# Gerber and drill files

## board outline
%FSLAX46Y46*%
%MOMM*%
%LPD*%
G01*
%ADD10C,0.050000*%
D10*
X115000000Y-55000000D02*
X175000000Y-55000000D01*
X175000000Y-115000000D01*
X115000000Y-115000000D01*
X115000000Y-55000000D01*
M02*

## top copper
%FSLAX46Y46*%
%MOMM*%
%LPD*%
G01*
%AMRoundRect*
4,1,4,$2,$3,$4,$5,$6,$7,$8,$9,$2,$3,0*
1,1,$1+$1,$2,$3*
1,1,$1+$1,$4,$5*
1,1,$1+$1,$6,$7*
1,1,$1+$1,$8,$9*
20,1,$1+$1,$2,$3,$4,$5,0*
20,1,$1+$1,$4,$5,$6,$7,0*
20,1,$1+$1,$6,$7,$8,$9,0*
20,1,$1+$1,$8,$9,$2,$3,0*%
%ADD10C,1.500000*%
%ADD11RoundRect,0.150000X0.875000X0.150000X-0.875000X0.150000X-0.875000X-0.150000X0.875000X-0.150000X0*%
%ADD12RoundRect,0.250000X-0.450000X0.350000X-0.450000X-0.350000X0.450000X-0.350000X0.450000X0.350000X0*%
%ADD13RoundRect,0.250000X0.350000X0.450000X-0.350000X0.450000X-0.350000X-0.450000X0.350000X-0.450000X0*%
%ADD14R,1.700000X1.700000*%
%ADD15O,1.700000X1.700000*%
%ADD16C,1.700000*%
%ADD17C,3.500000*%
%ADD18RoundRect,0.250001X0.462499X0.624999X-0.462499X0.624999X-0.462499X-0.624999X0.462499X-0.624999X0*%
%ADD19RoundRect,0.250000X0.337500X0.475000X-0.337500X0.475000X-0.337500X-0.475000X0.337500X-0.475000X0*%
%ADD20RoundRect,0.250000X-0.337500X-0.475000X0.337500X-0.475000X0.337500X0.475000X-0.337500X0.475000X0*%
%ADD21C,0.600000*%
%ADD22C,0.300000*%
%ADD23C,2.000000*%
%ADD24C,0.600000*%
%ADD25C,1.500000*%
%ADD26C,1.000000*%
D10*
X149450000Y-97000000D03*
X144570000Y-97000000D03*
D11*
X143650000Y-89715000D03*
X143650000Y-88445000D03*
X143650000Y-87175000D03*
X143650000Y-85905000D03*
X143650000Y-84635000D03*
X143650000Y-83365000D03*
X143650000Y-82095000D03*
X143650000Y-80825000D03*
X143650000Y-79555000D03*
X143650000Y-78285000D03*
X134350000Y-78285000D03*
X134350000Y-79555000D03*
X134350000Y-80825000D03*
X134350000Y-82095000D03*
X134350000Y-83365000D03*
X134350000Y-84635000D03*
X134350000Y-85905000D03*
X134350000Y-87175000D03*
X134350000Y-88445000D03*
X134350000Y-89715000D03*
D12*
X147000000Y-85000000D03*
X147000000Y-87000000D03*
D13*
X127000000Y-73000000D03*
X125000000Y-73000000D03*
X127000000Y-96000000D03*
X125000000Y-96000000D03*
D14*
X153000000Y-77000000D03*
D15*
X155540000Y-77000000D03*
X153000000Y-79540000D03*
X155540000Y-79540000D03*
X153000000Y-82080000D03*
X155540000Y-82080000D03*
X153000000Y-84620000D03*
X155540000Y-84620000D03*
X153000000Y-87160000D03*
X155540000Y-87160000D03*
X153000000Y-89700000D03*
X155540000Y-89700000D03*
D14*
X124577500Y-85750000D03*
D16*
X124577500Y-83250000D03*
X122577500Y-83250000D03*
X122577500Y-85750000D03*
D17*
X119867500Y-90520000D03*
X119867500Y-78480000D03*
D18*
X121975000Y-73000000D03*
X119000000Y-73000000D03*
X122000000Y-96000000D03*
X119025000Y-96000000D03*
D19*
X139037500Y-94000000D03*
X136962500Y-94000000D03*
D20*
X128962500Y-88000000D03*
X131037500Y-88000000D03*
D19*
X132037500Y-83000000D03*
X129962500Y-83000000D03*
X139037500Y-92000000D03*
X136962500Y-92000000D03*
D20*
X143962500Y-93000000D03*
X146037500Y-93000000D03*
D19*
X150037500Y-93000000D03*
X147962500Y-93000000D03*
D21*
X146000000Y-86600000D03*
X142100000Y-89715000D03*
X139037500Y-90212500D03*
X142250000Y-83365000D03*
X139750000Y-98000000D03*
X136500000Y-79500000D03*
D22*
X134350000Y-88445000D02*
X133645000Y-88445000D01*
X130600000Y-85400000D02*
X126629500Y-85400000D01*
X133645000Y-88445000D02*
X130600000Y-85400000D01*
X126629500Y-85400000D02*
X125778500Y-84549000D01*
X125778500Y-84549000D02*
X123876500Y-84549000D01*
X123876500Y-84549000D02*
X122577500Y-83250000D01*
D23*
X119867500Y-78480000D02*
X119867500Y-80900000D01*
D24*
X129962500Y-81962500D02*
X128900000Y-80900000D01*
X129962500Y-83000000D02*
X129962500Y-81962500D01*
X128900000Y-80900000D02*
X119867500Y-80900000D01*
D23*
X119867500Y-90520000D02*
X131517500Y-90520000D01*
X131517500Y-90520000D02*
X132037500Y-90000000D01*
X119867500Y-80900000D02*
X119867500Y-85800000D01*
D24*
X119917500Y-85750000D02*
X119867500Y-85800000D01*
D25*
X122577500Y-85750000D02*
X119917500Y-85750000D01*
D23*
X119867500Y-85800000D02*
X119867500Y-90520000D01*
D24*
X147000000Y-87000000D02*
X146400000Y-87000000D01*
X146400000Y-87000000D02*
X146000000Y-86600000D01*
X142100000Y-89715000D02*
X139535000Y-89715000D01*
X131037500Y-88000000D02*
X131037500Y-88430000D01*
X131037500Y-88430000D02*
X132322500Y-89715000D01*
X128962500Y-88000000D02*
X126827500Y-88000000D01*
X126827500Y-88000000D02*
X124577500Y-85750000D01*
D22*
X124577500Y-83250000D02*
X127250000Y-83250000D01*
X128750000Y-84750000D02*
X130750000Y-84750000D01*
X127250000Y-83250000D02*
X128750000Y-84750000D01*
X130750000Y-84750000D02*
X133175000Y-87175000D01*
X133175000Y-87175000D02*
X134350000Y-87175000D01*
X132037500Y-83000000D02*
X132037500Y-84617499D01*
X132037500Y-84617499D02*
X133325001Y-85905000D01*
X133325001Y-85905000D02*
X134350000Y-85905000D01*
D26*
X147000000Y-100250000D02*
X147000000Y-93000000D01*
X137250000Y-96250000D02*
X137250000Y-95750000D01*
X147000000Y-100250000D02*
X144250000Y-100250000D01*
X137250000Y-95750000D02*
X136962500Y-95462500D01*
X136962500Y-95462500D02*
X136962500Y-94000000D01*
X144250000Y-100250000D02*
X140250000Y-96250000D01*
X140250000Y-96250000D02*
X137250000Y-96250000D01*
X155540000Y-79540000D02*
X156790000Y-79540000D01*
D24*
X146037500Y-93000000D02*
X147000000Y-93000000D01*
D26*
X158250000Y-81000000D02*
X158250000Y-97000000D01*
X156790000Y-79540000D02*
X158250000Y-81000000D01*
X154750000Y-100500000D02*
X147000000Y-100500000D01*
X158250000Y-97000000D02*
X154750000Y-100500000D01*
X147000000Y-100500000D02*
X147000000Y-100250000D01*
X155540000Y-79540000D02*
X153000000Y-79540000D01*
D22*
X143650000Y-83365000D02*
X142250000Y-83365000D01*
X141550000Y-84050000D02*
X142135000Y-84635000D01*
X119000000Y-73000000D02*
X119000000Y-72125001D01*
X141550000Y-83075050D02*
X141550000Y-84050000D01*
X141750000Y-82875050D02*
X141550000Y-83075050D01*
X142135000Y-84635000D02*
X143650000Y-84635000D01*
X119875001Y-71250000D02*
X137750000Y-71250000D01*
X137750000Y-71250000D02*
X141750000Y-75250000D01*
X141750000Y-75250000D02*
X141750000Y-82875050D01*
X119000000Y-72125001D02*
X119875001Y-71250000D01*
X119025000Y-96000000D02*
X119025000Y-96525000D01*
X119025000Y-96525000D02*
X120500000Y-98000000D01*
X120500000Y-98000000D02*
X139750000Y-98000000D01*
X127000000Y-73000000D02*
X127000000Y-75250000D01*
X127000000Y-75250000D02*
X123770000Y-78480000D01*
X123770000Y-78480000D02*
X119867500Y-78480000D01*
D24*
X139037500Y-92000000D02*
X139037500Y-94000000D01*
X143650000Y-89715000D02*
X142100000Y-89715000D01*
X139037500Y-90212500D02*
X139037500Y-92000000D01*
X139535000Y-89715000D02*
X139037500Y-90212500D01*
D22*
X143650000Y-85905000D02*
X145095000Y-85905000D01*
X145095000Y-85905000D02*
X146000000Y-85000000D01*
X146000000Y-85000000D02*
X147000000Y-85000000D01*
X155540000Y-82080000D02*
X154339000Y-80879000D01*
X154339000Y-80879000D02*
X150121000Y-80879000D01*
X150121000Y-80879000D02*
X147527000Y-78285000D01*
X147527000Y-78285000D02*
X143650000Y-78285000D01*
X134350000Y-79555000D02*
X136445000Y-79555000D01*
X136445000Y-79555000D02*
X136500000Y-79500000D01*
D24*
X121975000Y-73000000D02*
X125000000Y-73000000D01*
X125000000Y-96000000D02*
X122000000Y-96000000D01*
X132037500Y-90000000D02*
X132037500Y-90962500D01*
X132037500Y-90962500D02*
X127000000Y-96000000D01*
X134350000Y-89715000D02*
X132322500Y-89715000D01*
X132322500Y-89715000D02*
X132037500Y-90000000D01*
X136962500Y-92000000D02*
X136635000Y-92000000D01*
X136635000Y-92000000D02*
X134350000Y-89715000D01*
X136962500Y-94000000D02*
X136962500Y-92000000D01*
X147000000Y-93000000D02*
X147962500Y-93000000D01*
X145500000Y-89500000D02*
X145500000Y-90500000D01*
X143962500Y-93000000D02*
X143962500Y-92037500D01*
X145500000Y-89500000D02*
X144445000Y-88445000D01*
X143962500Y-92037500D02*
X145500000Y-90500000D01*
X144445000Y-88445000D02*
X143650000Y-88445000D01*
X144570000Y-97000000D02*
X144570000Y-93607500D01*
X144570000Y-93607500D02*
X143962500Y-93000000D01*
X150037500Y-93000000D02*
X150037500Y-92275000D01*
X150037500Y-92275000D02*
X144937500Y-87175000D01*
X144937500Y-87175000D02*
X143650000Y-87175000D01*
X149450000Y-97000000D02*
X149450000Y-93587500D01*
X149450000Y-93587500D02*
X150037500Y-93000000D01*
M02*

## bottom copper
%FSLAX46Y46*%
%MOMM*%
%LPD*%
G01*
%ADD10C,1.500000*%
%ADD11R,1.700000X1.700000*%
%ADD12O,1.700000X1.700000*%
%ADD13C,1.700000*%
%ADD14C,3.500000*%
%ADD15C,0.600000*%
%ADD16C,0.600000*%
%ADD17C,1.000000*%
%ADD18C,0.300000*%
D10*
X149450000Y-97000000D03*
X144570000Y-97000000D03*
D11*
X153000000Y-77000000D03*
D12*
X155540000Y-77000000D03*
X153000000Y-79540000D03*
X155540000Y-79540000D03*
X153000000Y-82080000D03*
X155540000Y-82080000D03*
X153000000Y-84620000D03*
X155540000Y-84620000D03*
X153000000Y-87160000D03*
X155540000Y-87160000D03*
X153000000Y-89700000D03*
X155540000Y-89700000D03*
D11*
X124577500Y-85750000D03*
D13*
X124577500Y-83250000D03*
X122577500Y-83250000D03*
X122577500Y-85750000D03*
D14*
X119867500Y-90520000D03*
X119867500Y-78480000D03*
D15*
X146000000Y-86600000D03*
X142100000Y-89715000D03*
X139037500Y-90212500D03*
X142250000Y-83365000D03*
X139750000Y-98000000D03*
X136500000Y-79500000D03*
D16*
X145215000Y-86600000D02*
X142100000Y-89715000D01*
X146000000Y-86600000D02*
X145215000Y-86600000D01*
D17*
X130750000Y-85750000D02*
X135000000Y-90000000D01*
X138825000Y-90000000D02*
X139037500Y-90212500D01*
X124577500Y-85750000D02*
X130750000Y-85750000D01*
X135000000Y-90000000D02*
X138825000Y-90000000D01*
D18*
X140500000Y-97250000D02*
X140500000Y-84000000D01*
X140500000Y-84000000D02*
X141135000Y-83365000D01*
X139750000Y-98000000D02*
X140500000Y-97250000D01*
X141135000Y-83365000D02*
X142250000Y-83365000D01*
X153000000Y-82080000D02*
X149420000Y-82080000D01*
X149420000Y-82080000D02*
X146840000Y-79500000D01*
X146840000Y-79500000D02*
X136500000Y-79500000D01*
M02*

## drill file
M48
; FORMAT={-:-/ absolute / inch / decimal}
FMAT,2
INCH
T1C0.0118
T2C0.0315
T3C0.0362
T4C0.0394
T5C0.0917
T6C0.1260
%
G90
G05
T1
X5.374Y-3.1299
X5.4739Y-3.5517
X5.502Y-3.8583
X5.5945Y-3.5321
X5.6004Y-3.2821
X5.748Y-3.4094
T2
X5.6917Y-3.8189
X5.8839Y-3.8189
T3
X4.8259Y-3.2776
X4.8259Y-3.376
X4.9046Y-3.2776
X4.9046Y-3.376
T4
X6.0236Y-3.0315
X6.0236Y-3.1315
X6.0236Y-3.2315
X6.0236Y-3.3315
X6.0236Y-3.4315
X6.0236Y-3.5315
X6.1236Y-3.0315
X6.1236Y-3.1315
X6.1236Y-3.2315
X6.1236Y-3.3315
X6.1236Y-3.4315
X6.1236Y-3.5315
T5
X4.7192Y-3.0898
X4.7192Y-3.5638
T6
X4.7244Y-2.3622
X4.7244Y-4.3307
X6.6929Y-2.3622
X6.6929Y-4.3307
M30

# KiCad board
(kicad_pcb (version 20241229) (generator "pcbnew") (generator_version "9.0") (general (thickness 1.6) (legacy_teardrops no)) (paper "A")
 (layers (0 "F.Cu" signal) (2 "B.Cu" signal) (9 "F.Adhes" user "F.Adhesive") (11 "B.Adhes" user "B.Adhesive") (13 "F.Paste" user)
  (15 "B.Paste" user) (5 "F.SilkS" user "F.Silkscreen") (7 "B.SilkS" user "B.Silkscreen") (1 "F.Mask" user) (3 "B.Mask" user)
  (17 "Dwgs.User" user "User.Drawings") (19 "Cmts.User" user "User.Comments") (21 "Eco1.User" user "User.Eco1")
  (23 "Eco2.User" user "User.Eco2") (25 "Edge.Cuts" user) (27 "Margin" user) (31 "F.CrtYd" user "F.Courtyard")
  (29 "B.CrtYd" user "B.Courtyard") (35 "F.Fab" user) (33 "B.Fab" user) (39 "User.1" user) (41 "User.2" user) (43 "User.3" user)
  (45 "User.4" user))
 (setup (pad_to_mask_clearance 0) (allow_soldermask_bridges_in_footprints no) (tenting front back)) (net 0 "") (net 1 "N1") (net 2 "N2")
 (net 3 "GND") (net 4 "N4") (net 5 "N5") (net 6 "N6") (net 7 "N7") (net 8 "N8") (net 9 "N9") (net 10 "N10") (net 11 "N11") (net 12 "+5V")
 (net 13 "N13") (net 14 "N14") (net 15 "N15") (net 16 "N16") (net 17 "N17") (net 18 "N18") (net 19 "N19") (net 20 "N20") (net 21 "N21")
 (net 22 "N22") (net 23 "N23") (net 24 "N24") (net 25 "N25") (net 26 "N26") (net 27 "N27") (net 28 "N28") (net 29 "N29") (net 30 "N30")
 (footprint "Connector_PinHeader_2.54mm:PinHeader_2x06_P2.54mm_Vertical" (layer "F.Cu") (at 153 77)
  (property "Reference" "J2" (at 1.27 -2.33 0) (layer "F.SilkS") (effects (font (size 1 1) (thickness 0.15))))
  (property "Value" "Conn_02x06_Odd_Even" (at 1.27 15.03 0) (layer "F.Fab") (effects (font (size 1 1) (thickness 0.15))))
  (pad "1" thru_hole rect (at 0 0) (size 1.7 1.7) (drill 1) (layers "*.Cu" "*.Mask") (remove_unused_layers no) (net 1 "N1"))
  (pad "2" thru_hole oval (at 2.54 0) (size 1.7 1.7) (drill 1) (layers "*.Cu" "*.Mask") (remove_unused_layers no) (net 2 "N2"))
  (pad "3" thru_hole oval (at 0 2.54) (size 1.7 1.7) (drill 1) (layers "*.Cu" "*.Mask") (remove_unused_layers no) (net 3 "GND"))
  (pad "4" thru_hole oval (at 2.54 2.54) (size 1.7 1.7) (drill 1) (layers "*.Cu" "*.Mask") (remove_unused_layers no) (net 3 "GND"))
  (pad "5" thru_hole oval (at 0 5.08) (size 1.7 1.7) (drill 1) (layers "*.Cu" "*.Mask") (remove_unused_layers no) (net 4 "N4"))
  (pad "6" thru_hole oval (at 2.54 5.08) (size 1.7 1.7) (drill 1) (layers "*.Cu" "*.Mask") (remove_unused_layers no) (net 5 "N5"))
  (pad "7" thru_hole oval (at 0 7.62) (size 1.7 1.7) (drill 1) (layers "*.Cu" "*.Mask") (remove_unused_layers no) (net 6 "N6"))
  (pad "8" thru_hole oval (at 2.54 7.62) (size 1.7 1.7) (drill 1) (layers "*.Cu" "*.Mask") (remove_unused_layers no) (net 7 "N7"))
  (pad "9" thru_hole oval (at 0 10.16) (size 1.7 1.7) (drill 1) (layers "*.Cu" "*.Mask") (remove_unused_layers no) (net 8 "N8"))
  (pad "10" thru_hole oval (at 2.54 10.16) (size 1.7 1.7) (drill 1) (layers "*.Cu" "*.Mask") (remove_unused_layers no) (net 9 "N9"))
  (pad "11" thru_hole oval (at 0 12.7) (size 1.7 1.7) (drill 1) (layers "*.Cu" "*.Mask") (remove_unused_layers no) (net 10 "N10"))
  (pad "12" thru_hole oval (at 2.54 12.7) (size 1.7 1.7) (drill 1) (layers "*.Cu" "*.Mask") (remove_unused_layers no) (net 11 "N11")))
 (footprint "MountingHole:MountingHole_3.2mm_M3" (layer "F.Cu") (at 120 110)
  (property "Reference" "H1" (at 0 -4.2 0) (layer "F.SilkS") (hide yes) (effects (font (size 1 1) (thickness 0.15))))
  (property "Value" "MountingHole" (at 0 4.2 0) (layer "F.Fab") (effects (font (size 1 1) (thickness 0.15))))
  (pad "" np_thru_hole circle (at 0 0) (size 3.2 3.2) (drill 3.2) (layers "*.Cu" "*.Mask")))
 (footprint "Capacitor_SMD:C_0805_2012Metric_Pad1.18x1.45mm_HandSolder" (layer "F.Cu") (at 130 88)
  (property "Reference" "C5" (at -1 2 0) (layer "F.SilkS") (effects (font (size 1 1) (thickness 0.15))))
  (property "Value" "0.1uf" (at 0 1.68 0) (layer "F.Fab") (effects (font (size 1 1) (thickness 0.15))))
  (pad "1" smd roundrect (at -1.0375 0) (size 1.175 1.45) (layers "F.Cu" "F.Mask" "F.Paste") (roundrect_rratio 0.212766) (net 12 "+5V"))
  (pad "2" smd roundrect (at 1.0375 0) (size 1.175 1.45) (layers "F.Cu" "F.Mask" "F.Paste") (roundrect_rratio 0.212766) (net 3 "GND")))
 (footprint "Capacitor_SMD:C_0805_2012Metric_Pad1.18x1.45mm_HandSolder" (layer "F.Cu") (at 138 94 180)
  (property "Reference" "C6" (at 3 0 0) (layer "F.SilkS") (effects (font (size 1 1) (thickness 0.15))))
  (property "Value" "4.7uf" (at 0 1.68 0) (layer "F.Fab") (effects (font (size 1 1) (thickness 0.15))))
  (pad "1" smd roundrect (at -1.0375 0 180) (size 1.175 1.45) (layers "F.Cu" "F.Mask" "F.Paste") (roundrect_rratio 0.212766) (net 12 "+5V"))
  (pad "2" smd roundrect (at 1.0375 0 180) (size 1.175 1.45) (layers "F.Cu" "F.Mask" "F.Paste") (roundrect_rratio 0.212766) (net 3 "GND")))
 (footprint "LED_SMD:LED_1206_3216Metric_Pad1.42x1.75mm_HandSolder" (layer "F.Cu") (at 120.5125 96 180)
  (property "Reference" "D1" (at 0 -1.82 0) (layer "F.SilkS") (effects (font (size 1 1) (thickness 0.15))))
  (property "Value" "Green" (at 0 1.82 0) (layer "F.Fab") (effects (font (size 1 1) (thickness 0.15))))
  (pad "1" smd roundrect (at -1.4875 0 180) (size 1.425 1.75) (layers "F.Cu" "F.Mask" "F.Paste") (roundrect_rratio 0.175439) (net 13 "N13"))
  (pad "2" smd roundrect (at 1.4875 0 180) (size 1.425 1.75) (layers "F.Cu" "F.Mask" "F.Paste") (roundrect_rratio 0.175439) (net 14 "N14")))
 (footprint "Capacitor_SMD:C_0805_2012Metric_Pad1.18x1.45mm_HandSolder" (layer "F.Cu") (at 138 92 180)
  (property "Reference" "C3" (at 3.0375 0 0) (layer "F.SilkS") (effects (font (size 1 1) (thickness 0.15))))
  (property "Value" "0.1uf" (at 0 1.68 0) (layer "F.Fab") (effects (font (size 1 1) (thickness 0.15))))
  (pad "1" smd roundrect (at -1.0375 0 180) (size 1.175 1.45) (layers "F.Cu" "F.Mask" "F.Paste") (roundrect_rratio 0.212766) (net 12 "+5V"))
  (pad "2" smd roundrect (at 1.0375 0 180) (size 1.175 1.45) (layers "F.Cu" "F.Mask" "F.Paste") (roundrect_rratio 0.212766) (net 3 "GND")))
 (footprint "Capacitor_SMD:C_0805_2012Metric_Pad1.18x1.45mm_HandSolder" (layer "F.Cu") (at 131 83 180)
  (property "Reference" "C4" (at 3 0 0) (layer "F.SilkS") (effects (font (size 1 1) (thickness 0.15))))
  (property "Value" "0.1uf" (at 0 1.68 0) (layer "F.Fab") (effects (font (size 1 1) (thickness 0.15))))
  (pad "1" smd roundrect (at -1.0375 0 180) (size 1.175 1.45) (layers "F.Cu" "F.Mask" "F.Paste") (roundrect_rratio 0.212766) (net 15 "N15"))
  (pad "2" smd roundrect (at 1.0375 0 180) (size 1.175 1.45) (layers "F.Cu" "F.Mask" "F.Paste") (roundrect_rratio 0.212766) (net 3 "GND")))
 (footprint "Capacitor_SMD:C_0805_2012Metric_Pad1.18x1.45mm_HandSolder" (layer "F.Cu") (at 145 93)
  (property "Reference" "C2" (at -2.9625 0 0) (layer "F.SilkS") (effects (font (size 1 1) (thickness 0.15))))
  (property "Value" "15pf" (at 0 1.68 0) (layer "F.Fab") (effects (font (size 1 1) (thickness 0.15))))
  (pad "1" smd roundrect (at -1.0375 0) (size 1.175 1.45) (layers "F.Cu" "F.Mask" "F.Paste") (roundrect_rratio 0.212766) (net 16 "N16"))
  (pad "2" smd roundrect (at 1.0375 0) (size 1.175 1.45) (layers "F.Cu" "F.Mask" "F.Paste") (roundrect_rratio 0.212766) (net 3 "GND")))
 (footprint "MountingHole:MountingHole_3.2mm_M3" (layer "F.Cu") (at 170 110)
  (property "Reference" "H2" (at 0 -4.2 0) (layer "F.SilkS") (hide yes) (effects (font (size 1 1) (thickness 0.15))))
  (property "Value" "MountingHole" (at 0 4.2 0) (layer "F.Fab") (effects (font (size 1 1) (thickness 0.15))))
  (pad "" np_thru_hole circle (at 0 0) (size 3.2 3.2) (drill 3.2) (layers "*.Cu" "*.Mask")))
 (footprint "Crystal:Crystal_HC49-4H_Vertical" (layer "F.Cu") (at 149.45 97 180)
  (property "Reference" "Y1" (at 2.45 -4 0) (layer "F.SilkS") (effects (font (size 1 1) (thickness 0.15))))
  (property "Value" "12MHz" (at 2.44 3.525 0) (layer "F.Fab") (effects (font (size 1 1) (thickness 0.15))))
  (pad "1" thru_hole circle (at 0 0 180) (size 1.5 1.5) (drill 0.8) (layers "*.Cu" "*.Mask") (remove_unused_layers no) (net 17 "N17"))
  (pad "2" thru_hole circle (at 4.88 0 180) (size 1.5 1.5) (drill 0.8) (layers "*.Cu" "*.Mask") (remove_unused_layers no) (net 16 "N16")))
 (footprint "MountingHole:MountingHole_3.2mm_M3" (layer "F.Cu") (at 170 60)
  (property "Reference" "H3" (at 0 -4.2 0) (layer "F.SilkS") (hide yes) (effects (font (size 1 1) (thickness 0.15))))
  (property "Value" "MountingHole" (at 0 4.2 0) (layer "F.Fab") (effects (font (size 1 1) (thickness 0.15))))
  (pad "" np_thru_hole circle (at 0 0) (size 3.2 3.2) (drill 3.2) (layers "*.Cu" "*.Mask")))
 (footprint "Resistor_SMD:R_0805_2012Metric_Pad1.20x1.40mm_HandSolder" (layer "F.Cu") (at 126 73 180)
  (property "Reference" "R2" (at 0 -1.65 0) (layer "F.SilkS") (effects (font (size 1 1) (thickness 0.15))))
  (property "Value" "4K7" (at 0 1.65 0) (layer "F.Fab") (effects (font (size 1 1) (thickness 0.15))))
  (pad "1" smd roundrect (at -1 0 180) (size 1.2 1.4) (layers "F.Cu" "F.Mask" "F.Paste") (roundrect_rratio 0.208333) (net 3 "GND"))
  (pad "2" smd roundrect (at 1 0 180) (size 1.2 1.4) (layers "F.Cu" "F.Mask" "F.Paste") (roundrect_rratio 0.208333) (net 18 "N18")))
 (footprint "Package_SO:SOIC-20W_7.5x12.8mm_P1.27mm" (layer "F.Cu") (at 139 84 180)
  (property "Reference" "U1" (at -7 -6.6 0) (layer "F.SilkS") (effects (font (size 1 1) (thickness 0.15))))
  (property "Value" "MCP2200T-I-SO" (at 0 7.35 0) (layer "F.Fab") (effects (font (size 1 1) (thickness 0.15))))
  (pad "1" smd roundrect (at -4.65 -5.715 180) (size 2.05 0.6) (layers "F.Cu" "F.Mask" "F.Paste") (roundrect_rratio 0.25) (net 12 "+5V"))
  (pad "2" smd roundrect (at -4.65 -4.445 180) (size 2.05 0.6) (layers "F.Cu" "F.Mask" "F.Paste") (roundrect_rratio 0.25) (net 16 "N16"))
  (pad "3" smd roundrect (at -4.65 -3.175 180) (size 2.05 0.6) (layers "F.Cu" "F.Mask" "F.Paste") (roundrect_rratio 0.25) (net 17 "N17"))
  (pad "4" smd roundrect (at -4.65 -1.905 180) (size 2.05 0.6) (layers "F.Cu" "F.Mask" "F.Paste") (roundrect_rratio 0.25) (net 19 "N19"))
  (pad "5" smd roundrect (at -4.65 -0.635 180) (size 2.05 0.6) (layers "F.Cu" "F.Mask" "F.Paste") (roundrect_rratio 0.25) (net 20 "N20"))
  (pad "6" smd roundrect (at -4.65 0.635 180) (size 2.05 0.6) (layers "F.Cu" "F.Mask" "F.Paste") (roundrect_rratio 0.25) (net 14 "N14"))
  (pad "7" smd roundrect (at -4.65 1.905 180) (size 2.05 0.6) (layers "F.Cu" "F.Mask" "F.Paste") (roundrect_rratio 0.25) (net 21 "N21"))
  (pad "8" smd roundrect (at -4.65 3.175 180) (size 2.05 0.6) (layers "F.Cu" "F.Mask" "F.Paste") (roundrect_rratio 0.25) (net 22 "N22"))
  (pad "9" smd roundrect (at -4.65 4.445 180) (size 2.05 0.6) (layers "F.Cu" "F.Mask" "F.Paste") (roundrect_rratio 0.25) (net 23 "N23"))
  (pad "10" smd roundrect (at -4.65 5.715 180) (size 2.05 0.6) (layers "F.Cu" "F.Mask" "F.Paste") (roundrect_rratio 0.25) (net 5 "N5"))
  (pad "11" smd roundrect (at 4.65 5.715 180) (size 2.05 0.6) (layers "F.Cu" "F.Mask" "F.Paste") (roundrect_rratio 0.25) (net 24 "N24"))
  (pad "12" smd roundrect (at 4.65 4.445 180) (size 2.05 0.6) (layers "F.Cu" "F.Mask" "F.Paste") (roundrect_rratio 0.25) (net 4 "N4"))
  (pad "13" smd roundrect (at 4.65 3.175 180) (size 2.05 0.6) (layers "F.Cu" "F.Mask" "F.Paste") (roundrect_rratio 0.25) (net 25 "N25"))
  (pad "14" smd roundrect (at 4.65 1.905 180) (size 2.05 0.6) (layers "F.Cu" "F.Mask" "F.Paste") (roundrect_rratio 0.25) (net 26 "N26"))
  (pad "15" smd roundrect (at 4.65 0.635 180) (size 2.05 0.6) (layers "F.Cu" "F.Mask" "F.Paste") (roundrect_rratio 0.25) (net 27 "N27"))
  (pad "16" smd roundrect (at 4.65 -0.635 180) (size 2.05 0.6) (layers "F.Cu" "F.Mask" "F.Paste") (roundrect_rratio 0.25) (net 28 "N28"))
  (pad "17" smd roundrect (at 4.65 -1.905 180) (size 2.05 0.6) (layers "F.Cu" "F.Mask" "F.Paste") (roundrect_rratio 0.25) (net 15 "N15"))
  (pad "18" smd roundrect (at 4.65 -3.175 180) (size 2.05 0.6) (layers "F.Cu" "F.Mask" "F.Paste") (roundrect_rratio 0.25) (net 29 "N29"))
  (pad "19" smd roundrect (at 4.65 -4.445 180) (size 2.05 0.6) (layers "F.Cu" "F.Mask" "F.Paste") (roundrect_rratio 0.25) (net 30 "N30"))
  (pad "20" smd roundrect (at 4.65 -5.715 180) (size 2.05 0.6) (layers "F.Cu" "F.Mask" "F.Paste") (roundrect_rratio 0.25) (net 3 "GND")))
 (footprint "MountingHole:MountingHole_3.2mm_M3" (layer "F.Cu") (at 120 60)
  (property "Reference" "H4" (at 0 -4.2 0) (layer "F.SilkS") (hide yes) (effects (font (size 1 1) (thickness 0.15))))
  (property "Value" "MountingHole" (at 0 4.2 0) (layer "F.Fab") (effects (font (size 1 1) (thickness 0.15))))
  (pad "" np_thru_hole circle (at 0 0) (size 3.2 3.2) (drill 3.2) (layers "*.Cu" "*.Mask")))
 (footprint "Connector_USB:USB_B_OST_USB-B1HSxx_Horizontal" (layer "F.Cu") (at 124.5775 85.75 180)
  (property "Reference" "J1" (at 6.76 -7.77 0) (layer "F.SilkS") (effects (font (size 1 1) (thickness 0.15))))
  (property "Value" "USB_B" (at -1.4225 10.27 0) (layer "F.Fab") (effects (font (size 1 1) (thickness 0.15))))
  (pad "1" thru_hole rect (at 0 0 180) (size 1.7 1.7) (drill 0.92) (layers "*.Cu" "*.Mask") (remove_unused_layers no) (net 12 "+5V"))
  (pad "2" thru_hole circle (at 0 2.5 180) (size 1.7 1.7) (drill 0.92) (layers "*.Cu" "*.Mask") (remove_unused_layers no) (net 29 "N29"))
  (pad "3" thru_hole circle (at 2 2.5 180) (size 1.7 1.7) (drill 0.92) (layers "*.Cu" "*.Mask") (remove_unused_layers no) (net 30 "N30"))
  (pad "4" thru_hole circle (at 2 0 180) (size 1.7 1.7) (drill 0.92) (layers "*.Cu" "*.Mask") (remove_unused_layers no) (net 3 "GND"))
  (pad "5" thru_hole circle (at 4.71 -4.77 180) (size 3.5 3.5) (drill 2.33) (layers "*.Cu" "*.Mask") (remove_unused_layers no) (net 3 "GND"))
  (pad "5" thru_hole circle (at 4.71 7.27 180) (size 3.5 3.5) (drill 2.33) (layers "*.Cu" "*.Mask") (remove_unused_layers no) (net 3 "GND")))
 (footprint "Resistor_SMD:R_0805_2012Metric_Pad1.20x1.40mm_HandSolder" (layer "F.Cu") (at 147 86 -90)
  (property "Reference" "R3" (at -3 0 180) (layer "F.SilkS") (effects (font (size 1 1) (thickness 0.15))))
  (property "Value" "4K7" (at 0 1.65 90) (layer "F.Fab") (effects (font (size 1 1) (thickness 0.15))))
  (pad "1" smd roundrect (at -1 0 270) (size 1.2 1.4) (layers "F.Cu" "F.Mask" "F.Paste") (roundrect_rratio 0.208333) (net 19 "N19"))
  (pad "2" smd roundrect (at 1 0 270) (size 1.2 1.4) (layers "F.Cu" "F.Mask" "F.Paste") (roundrect_rratio 0.208333) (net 12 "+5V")))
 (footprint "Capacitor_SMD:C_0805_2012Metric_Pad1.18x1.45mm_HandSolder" (layer "F.Cu") (at 149 93 180)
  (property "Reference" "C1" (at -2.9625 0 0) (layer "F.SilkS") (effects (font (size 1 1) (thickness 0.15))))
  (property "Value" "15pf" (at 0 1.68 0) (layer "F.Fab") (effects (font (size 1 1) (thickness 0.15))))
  (pad "1" smd roundrect (at -1.0375 0 180) (size 1.175 1.45) (layers "F.Cu" "F.Mask" "F.Paste") (roundrect_rratio 0.212766) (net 17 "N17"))
  (pad "2" smd roundrect (at 1.0375 0 180) (size 1.175 1.45) (layers "F.Cu" "F.Mask" "F.Paste") (roundrect_rratio 0.212766) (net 3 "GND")))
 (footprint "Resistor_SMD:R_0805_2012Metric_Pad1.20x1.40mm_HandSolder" (layer "F.Cu") (at 126 96 180)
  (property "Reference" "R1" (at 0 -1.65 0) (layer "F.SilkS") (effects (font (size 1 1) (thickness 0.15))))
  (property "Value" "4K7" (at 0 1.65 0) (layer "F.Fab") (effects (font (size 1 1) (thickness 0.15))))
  (pad "1" smd roundrect (at -1 0 180) (size 1.2 1.4) (layers "F.Cu" "F.Mask" "F.Paste") (roundrect_rratio 0.208333) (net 3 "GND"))
  (pad "2" smd roundrect (at 1 0 180) (size 1.2 1.4) (layers "F.Cu" "F.Mask" "F.Paste") (roundrect_rratio 0.208333) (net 13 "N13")))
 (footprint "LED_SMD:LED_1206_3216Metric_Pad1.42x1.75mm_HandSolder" (layer "F.Cu") (at 120.4875 73 180)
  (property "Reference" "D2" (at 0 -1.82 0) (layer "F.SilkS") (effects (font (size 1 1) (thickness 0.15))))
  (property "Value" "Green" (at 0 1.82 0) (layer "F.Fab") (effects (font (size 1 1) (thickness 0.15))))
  (pad "1" smd roundrect (at -1.4875 0 180) (size 1.425 1.75) (layers "F.Cu" "F.Mask" "F.Paste") (roundrect_rratio 0.175439) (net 18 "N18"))
  (pad "2" smd roundrect (at 1.4875 0 180) (size 1.425 1.75) (layers "F.Cu" "F.Mask" "F.Paste") (roundrect_rratio 0.175439) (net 20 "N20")))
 (gr_rect (start 115 55) (end 175 115) (stroke (width 0.05) (type default)) (fill no) (layer "Edge.Cuts"))
 (segment (start 131.5175 90.52) (end 132.0375 90) (width 2) (layer "F.Cu") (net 3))
 (segment (start 132.3225 89.715) (end 132.0375 90) (width 0.6) (layer "F.Cu") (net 3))
 (segment (start 132.0375 90) (end 132.0375 90.9625) (width 0.6) (layer "F.Cu") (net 3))
 (segment (start 132.0375 90.9625) (end 127 96) (width 0.6) (layer "F.Cu") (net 3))
 (segment (start 129.9625 81.9625) (end 128.9 80.9) (width 0.6) (layer "F.Cu") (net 3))
 (segment (start 137.25 95.75) (end 136.9625 95.4625) (width 1) (layer "F.Cu") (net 3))
 (segment (start 119.8675 78.48) (end 119.8675 80.9) (width 2) (layer "F.Cu") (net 3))
 (segment (start 146.0375 93) (end 147 93) (width 0.6) (layer "F.Cu") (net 3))
 (segment (start 147 100.25) (end 144.25 100.25) (width 1) (layer "F.Cu") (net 3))
 (segment (start 147 100.25) (end 147 93) (width 1) (layer "F.Cu") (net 3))
 (segment (start 119.8675 80.9) (end 119.8675 85.8) (width 2) (layer "F.Cu") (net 3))
 (segment (start 158.25 81) (end 158.25 97) (width 1) (layer "F.Cu") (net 3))
 (segment (start 156.79 79.54) (end 158.25 81) (width 1) (layer "F.Cu") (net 3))
 (segment (start 140.25 96.25) (end 137.25 96.25) (width 1) (layer "F.Cu") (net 3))
 (segment (start 136.9625 95.4625) (end 136.9625 94) (width 1) (layer "F.Cu") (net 3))
 (segment (start 147 100.5) (end 147 100.25) (width 1) (layer "F.Cu") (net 3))
 (segment (start 155.54 79.54) (end 153 79.54) (width 1) (layer "F.Cu") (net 3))
 (segment (start 122.5775 85.75) (end 119.9175 85.75) (width 1.5) (layer "F.Cu") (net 3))
 (segment (start 144.25 100.25) (end 140.25 96.25) (width 1) (layer "F.Cu") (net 3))
 (segment (start 131.0375 88) (end 131.0375 88.43) (width 0.6) (layer "F.Cu") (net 3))
 (segment (start 128.9 80.9) (end 119.8675 80.9) (width 0.6) (layer "F.Cu") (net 3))
 (segment (start 129.9625 83) (end 129.9625 81.9625) (width 0.6) (layer "F.Cu") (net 3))
 (segment (start 136.9625 94) (end 136.9625 92) (width 0.6) (layer "F.Cu") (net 3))
 (segment (start 137.25 96.25) (end 137.25 95.75) (width 1) (layer "F.Cu") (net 3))
 (segment (start 155.54 79.54) (end 156.79 79.54) (width 1) (layer "F.Cu") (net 3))
 (segment (start 127 73) (end 127 75.25) (width 0.3) (layer "F.Cu") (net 3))
 (segment (start 119.8675 90.52) (end 131.5175 90.52) (width 2) (layer "F.Cu") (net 3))
 (segment (start 119.8675 85.8) (end 119.8675 90.52) (width 2) (layer "F.Cu") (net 3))
 (segment (start 158.25 97) (end 154.75 100.5) (width 1) (layer "F.Cu") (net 3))
 (segment (start 119.9175 85.75) (end 119.8675 85.8) (width 0.6) (layer "F.Cu") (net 3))
 (segment (start 131.0375 88.43) (end 132.3225 89.715) (width 0.6) (layer "F.Cu") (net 3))
 (segment (start 154.75 100.5) (end 147 100.5) (width 1) (layer "F.Cu") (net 3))
 (segment (start 134.35 89.715) (end 132.3225 89.715) (width 0.6) (layer "F.Cu") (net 3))
 (segment (start 123.77 78.48) (end 119.8675 78.48) (width 0.3) (layer "F.Cu") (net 3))
 (segment (start 136.635 92) (end 134.35 89.715) (width 0.6) (layer "F.Cu") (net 3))
 (segment (start 136.9625 92) (end 136.635 92) (width 0.6) (layer "F.Cu") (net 3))
 (segment (start 147 93) (end 147.9625 93) (width 0.6) (layer "F.Cu") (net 3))
 (segment (start 127 75.25) (end 123.77 78.48) (width 0.3) (layer "F.Cu") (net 3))
 (segment (start 149.45 93.5875) (end 150.0375 93) (width 0.6) (layer "F.Cu") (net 17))
 (segment (start 150.0375 93) (end 150.0375 92.275) (width 0.6) (layer "F.Cu") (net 17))
 (segment (start 144.9375 87.175) (end 143.65 87.175) (width 0.6) (layer "F.Cu") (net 17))
 (segment (start 150.0375 92.275) (end 144.9375 87.175) (width 0.6) (layer "F.Cu") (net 17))
 (segment (start 149.45 97) (end 149.45 93.5875) (width 0.6) (layer "F.Cu") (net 17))
 (segment (start 143.9625 92.0375) (end 145.5 90.5) (width 0.6) (layer "F.Cu") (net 16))
 (segment (start 145.5 89.5) (end 144.445 88.445) (width 0.6) (layer "F.Cu") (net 16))
 (segment (start 144.445 88.445) (end 143.65 88.445) (width 0.6) (layer "F.Cu") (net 16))
 (segment (start 145.5 89.5) (end 145.5 90.5) (width 0.6) (layer "F.Cu") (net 16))
 (segment (start 143.9625 93) (end 143.9625 92.0375) (width 0.6) (layer "F.Cu") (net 16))
 (segment (start 144.57 93.6075) (end 143.9625 93) (width 0.6) (layer "F.Cu") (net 16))
 (segment (start 144.57 97) (end 144.57 93.6075) (width 0.6) (layer "F.Cu") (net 16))
 (segment (start 143.65 89.715) (end 142.1 89.715) (width 0.6) (layer "F.Cu") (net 12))
 (segment (start 128.9625 88) (end 126.8275 88) (width 0.6) (layer "F.Cu") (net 12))
 (segment (start 146.4 87) (end 146 86.6) (width 0.6) (layer "F.Cu") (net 12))
 (segment (start 139.535 89.715) (end 139.0375 90.2125) (width 0.6) (layer "F.Cu") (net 12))
 (segment (start 147 87) (end 146.4 87) (width 0.6) (layer "F.Cu") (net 12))
 (segment (start 139.0375 92) (end 139.0375 94) (width 0.6) (layer "F.Cu") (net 12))
 (segment (start 126.8275 88) (end 124.5775 85.75) (width 0.6) (layer "F.Cu") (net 12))
 (segment (start 139.0375 90.2125) (end 139.0375 92) (width 0.6) (layer "F.Cu") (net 12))
 (segment (start 142.1 89.715) (end 139.535 89.715) (width 0.6) (layer "F.Cu") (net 12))
 (via (at 139.0375 90.2125) (size 0.6) (drill 0.3) (layers "F.Cu" "B.Cu") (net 12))
 (via (at 142.1 89.715) (size 0.6) (drill 0.3) (layers "F.Cu" "B.Cu") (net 12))
 (via (at 146 86.6) (size 0.6) (drill 0.3) (layers "F.Cu" "B.Cu") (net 12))
 (segment (start 124.5775 85.75) (end 130.75 85.75) (width 1) (layer "B.Cu") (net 12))
 (segment (start 146 86.6) (end 145.215 86.6) (width 0.6) (layer "B.Cu") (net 12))
 (segment (start 130.75 85.75) (end 135 90) (width 1) (layer "B.Cu") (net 12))
 (segment (start 135 90) (end 138.825 90) (width 1) (layer "B.Cu") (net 12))
 (segment (start 138.825 90) (end 139.0375 90.2125) (width 1) (layer "B.Cu") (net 12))
 (segment (start 145.215 86.6) (end 142.1 89.715) (width 0.6) (layer "B.Cu") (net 12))
 (segment (start 133.325001 85.905) (end 134.35 85.905) (width 0.3) (layer "F.Cu") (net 15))
 (segment (start 132.0375 84.617499) (end 133.325001 85.905) (width 0.3) (layer "F.Cu") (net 15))
 (segment (start 132.0375 83) (end 132.0375 84.617499) (width 0.3) (layer "F.Cu") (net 15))
 (segment (start 119.025 96.525) (end 120.5 98) (width 0.3) (layer "F.Cu") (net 14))
 (segment (start 119.025 96) (end 119.025 96.525) (width 0.3) (layer "F.Cu") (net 14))
 (segment (start 143.65 83.365) (end 142.25 83.365) (width 0.3) (layer "F.Cu") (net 14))
 (segment (start 120.5 98) (end 139.75 98) (width 0.3) (layer "F.Cu") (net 14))
 (via (at 139.75 98) (size 0.6) (drill 0.3) (layers "F.Cu" "B.Cu") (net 14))
 (via (at 142.25 83.365) (size 0.6) (drill 0.3) (layers "F.Cu" "B.Cu") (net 14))
 (segment (start 141.135 83.365) (end 142.25 83.365) (width 0.3) (layer "B.Cu") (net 14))
 (segment (start 140.5 97.25) (end 140.5 84) (width 0.3) (layer "B.Cu") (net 14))
 (segment (start 139.75 98) (end 140.5 97.25) (width 0.3) (layer "B.Cu") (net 14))
 (segment (start 140.5 84) (end 141.135 83.365) (width 0.3) (layer "B.Cu") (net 14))
 (segment (start 125 96) (end 122 96) (width 0.6) (layer "F.Cu") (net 13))
 (segment (start 121.975 73) (end 125 73) (width 0.6) (layer "F.Cu") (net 18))
 (segment (start 141.75 82.87505) (end 141.55 83.07505) (width 0.3) (layer "F.Cu") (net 20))
 (segment (start 119 72.125001) (end 119.875001 71.25) (width 0.3) (layer "F.Cu") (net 20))
 (segment (start 141.55 84.05) (end 142.135 84.635) (width 0.3) (layer "F.Cu") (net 20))
 (segment (start 141.75 75.25) (end 141.75 82.87505) (width 0.3) (layer "F.Cu") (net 20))
 (segment (start 119.875001 71.25) (end 137.75 71.25) (width 0.3) (layer "F.Cu") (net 20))
 (segment (start 137.75 71.25) (end 141.75 75.25) (width 0.3) (layer "F.Cu") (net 20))
 (segment (start 142.135 84.635) (end 143.65 84.635) (width 0.3) (layer "F.Cu") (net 20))
 (segment (start 119 73) (end 119 72.125001) (width 0.3) (layer "F.Cu") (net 20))
 (segment (start 141.55 83.07505) (end 141.55 84.05) (width 0.3) (layer "F.Cu") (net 20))
 (segment (start 127.25 83.25) (end 128.75 84.75) (width 0.3) (layer "F.Cu") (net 29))
 (segment (start 128.75 84.75) (end 130.75 84.75) (width 0.3) (layer "F.Cu") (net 29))
 (segment (start 133.175 87.175) (end 134.35 87.175) (width 0.3) (layer "F.Cu") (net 29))
 (segment (start 130.75 84.75) (end 133.175 87.175) (width 0.3) (layer "F.Cu") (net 29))
 (segment (start 124.5775 83.25) (end 127.25 83.25) (width 0.3) (layer "F.Cu") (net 29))
 (segment (start 130.6 85.4) (end 126.6295 85.4) (width 0.3) (layer "F.Cu") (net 30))
 (segment (start 123.8765 84.549) (end 122.5775 83.25) (width 0.3) (layer "F.Cu") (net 30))
 (segment (start 133.645 88.445) (end 130.6 85.4) (width 0.3) (layer "F.Cu") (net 30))
 (segment (start 125.7785 84.549) (end 123.8765 84.549) (width 0.3) (layer "F.Cu") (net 30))
 (segment (start 134.35 88.445) (end 133.645 88.445) (width 0.3) (layer "F.Cu") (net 30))
 (segment (start 126.6295 85.4) (end 125.7785 84.549) (width 0.3) (layer "F.Cu") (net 30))
 (segment (start 136.445 79.555) (end 136.5 79.5) (width 0.3) (layer "F.Cu") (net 4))
 (segment (start 134.35 79.555) (end 136.445 79.555) (width 0.3) (layer "F.Cu") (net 4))
 (via (at 136.5 79.5) (size 0.6) (drill 0.3) (layers "F.Cu" "B.Cu") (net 4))
 (segment (start 153 82.08) (end 149.42 82.08) (width 0.3) (layer "B.Cu") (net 4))
 (segment (start 149.42 82.08) (end 146.84 79.5) (width 0.3) (layer "B.Cu") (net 4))
 (segment (start 146.84 79.5) (end 136.5 79.5) (width 0.3) (layer "B.Cu") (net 4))
 (segment (start 155.54 82.08) (end 154.339 80.879) (width 0.3) (layer "F.Cu") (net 5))
 (segment (start 154.339 80.879) (end 150.121 80.879) (width 0.3) (layer "F.Cu") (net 5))
 (segment (start 150.121 80.879) (end 147.527 78.285) (width 0.3) (layer "F.Cu") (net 5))
 (segment (start 147.527 78.285) (end 143.65 78.285) (width 0.3) (layer "F.Cu") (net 5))
 (segment (start 143.65 85.905) (end 145.095 85.905) (width 0.3) (layer "F.Cu") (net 19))
 (segment (start 145.095 85.905) (end 146 85) (width 0.3) (layer "F.Cu") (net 19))
 (segment (start 146 85) (end 147 85) (width 0.3) (layer "F.Cu") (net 19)))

